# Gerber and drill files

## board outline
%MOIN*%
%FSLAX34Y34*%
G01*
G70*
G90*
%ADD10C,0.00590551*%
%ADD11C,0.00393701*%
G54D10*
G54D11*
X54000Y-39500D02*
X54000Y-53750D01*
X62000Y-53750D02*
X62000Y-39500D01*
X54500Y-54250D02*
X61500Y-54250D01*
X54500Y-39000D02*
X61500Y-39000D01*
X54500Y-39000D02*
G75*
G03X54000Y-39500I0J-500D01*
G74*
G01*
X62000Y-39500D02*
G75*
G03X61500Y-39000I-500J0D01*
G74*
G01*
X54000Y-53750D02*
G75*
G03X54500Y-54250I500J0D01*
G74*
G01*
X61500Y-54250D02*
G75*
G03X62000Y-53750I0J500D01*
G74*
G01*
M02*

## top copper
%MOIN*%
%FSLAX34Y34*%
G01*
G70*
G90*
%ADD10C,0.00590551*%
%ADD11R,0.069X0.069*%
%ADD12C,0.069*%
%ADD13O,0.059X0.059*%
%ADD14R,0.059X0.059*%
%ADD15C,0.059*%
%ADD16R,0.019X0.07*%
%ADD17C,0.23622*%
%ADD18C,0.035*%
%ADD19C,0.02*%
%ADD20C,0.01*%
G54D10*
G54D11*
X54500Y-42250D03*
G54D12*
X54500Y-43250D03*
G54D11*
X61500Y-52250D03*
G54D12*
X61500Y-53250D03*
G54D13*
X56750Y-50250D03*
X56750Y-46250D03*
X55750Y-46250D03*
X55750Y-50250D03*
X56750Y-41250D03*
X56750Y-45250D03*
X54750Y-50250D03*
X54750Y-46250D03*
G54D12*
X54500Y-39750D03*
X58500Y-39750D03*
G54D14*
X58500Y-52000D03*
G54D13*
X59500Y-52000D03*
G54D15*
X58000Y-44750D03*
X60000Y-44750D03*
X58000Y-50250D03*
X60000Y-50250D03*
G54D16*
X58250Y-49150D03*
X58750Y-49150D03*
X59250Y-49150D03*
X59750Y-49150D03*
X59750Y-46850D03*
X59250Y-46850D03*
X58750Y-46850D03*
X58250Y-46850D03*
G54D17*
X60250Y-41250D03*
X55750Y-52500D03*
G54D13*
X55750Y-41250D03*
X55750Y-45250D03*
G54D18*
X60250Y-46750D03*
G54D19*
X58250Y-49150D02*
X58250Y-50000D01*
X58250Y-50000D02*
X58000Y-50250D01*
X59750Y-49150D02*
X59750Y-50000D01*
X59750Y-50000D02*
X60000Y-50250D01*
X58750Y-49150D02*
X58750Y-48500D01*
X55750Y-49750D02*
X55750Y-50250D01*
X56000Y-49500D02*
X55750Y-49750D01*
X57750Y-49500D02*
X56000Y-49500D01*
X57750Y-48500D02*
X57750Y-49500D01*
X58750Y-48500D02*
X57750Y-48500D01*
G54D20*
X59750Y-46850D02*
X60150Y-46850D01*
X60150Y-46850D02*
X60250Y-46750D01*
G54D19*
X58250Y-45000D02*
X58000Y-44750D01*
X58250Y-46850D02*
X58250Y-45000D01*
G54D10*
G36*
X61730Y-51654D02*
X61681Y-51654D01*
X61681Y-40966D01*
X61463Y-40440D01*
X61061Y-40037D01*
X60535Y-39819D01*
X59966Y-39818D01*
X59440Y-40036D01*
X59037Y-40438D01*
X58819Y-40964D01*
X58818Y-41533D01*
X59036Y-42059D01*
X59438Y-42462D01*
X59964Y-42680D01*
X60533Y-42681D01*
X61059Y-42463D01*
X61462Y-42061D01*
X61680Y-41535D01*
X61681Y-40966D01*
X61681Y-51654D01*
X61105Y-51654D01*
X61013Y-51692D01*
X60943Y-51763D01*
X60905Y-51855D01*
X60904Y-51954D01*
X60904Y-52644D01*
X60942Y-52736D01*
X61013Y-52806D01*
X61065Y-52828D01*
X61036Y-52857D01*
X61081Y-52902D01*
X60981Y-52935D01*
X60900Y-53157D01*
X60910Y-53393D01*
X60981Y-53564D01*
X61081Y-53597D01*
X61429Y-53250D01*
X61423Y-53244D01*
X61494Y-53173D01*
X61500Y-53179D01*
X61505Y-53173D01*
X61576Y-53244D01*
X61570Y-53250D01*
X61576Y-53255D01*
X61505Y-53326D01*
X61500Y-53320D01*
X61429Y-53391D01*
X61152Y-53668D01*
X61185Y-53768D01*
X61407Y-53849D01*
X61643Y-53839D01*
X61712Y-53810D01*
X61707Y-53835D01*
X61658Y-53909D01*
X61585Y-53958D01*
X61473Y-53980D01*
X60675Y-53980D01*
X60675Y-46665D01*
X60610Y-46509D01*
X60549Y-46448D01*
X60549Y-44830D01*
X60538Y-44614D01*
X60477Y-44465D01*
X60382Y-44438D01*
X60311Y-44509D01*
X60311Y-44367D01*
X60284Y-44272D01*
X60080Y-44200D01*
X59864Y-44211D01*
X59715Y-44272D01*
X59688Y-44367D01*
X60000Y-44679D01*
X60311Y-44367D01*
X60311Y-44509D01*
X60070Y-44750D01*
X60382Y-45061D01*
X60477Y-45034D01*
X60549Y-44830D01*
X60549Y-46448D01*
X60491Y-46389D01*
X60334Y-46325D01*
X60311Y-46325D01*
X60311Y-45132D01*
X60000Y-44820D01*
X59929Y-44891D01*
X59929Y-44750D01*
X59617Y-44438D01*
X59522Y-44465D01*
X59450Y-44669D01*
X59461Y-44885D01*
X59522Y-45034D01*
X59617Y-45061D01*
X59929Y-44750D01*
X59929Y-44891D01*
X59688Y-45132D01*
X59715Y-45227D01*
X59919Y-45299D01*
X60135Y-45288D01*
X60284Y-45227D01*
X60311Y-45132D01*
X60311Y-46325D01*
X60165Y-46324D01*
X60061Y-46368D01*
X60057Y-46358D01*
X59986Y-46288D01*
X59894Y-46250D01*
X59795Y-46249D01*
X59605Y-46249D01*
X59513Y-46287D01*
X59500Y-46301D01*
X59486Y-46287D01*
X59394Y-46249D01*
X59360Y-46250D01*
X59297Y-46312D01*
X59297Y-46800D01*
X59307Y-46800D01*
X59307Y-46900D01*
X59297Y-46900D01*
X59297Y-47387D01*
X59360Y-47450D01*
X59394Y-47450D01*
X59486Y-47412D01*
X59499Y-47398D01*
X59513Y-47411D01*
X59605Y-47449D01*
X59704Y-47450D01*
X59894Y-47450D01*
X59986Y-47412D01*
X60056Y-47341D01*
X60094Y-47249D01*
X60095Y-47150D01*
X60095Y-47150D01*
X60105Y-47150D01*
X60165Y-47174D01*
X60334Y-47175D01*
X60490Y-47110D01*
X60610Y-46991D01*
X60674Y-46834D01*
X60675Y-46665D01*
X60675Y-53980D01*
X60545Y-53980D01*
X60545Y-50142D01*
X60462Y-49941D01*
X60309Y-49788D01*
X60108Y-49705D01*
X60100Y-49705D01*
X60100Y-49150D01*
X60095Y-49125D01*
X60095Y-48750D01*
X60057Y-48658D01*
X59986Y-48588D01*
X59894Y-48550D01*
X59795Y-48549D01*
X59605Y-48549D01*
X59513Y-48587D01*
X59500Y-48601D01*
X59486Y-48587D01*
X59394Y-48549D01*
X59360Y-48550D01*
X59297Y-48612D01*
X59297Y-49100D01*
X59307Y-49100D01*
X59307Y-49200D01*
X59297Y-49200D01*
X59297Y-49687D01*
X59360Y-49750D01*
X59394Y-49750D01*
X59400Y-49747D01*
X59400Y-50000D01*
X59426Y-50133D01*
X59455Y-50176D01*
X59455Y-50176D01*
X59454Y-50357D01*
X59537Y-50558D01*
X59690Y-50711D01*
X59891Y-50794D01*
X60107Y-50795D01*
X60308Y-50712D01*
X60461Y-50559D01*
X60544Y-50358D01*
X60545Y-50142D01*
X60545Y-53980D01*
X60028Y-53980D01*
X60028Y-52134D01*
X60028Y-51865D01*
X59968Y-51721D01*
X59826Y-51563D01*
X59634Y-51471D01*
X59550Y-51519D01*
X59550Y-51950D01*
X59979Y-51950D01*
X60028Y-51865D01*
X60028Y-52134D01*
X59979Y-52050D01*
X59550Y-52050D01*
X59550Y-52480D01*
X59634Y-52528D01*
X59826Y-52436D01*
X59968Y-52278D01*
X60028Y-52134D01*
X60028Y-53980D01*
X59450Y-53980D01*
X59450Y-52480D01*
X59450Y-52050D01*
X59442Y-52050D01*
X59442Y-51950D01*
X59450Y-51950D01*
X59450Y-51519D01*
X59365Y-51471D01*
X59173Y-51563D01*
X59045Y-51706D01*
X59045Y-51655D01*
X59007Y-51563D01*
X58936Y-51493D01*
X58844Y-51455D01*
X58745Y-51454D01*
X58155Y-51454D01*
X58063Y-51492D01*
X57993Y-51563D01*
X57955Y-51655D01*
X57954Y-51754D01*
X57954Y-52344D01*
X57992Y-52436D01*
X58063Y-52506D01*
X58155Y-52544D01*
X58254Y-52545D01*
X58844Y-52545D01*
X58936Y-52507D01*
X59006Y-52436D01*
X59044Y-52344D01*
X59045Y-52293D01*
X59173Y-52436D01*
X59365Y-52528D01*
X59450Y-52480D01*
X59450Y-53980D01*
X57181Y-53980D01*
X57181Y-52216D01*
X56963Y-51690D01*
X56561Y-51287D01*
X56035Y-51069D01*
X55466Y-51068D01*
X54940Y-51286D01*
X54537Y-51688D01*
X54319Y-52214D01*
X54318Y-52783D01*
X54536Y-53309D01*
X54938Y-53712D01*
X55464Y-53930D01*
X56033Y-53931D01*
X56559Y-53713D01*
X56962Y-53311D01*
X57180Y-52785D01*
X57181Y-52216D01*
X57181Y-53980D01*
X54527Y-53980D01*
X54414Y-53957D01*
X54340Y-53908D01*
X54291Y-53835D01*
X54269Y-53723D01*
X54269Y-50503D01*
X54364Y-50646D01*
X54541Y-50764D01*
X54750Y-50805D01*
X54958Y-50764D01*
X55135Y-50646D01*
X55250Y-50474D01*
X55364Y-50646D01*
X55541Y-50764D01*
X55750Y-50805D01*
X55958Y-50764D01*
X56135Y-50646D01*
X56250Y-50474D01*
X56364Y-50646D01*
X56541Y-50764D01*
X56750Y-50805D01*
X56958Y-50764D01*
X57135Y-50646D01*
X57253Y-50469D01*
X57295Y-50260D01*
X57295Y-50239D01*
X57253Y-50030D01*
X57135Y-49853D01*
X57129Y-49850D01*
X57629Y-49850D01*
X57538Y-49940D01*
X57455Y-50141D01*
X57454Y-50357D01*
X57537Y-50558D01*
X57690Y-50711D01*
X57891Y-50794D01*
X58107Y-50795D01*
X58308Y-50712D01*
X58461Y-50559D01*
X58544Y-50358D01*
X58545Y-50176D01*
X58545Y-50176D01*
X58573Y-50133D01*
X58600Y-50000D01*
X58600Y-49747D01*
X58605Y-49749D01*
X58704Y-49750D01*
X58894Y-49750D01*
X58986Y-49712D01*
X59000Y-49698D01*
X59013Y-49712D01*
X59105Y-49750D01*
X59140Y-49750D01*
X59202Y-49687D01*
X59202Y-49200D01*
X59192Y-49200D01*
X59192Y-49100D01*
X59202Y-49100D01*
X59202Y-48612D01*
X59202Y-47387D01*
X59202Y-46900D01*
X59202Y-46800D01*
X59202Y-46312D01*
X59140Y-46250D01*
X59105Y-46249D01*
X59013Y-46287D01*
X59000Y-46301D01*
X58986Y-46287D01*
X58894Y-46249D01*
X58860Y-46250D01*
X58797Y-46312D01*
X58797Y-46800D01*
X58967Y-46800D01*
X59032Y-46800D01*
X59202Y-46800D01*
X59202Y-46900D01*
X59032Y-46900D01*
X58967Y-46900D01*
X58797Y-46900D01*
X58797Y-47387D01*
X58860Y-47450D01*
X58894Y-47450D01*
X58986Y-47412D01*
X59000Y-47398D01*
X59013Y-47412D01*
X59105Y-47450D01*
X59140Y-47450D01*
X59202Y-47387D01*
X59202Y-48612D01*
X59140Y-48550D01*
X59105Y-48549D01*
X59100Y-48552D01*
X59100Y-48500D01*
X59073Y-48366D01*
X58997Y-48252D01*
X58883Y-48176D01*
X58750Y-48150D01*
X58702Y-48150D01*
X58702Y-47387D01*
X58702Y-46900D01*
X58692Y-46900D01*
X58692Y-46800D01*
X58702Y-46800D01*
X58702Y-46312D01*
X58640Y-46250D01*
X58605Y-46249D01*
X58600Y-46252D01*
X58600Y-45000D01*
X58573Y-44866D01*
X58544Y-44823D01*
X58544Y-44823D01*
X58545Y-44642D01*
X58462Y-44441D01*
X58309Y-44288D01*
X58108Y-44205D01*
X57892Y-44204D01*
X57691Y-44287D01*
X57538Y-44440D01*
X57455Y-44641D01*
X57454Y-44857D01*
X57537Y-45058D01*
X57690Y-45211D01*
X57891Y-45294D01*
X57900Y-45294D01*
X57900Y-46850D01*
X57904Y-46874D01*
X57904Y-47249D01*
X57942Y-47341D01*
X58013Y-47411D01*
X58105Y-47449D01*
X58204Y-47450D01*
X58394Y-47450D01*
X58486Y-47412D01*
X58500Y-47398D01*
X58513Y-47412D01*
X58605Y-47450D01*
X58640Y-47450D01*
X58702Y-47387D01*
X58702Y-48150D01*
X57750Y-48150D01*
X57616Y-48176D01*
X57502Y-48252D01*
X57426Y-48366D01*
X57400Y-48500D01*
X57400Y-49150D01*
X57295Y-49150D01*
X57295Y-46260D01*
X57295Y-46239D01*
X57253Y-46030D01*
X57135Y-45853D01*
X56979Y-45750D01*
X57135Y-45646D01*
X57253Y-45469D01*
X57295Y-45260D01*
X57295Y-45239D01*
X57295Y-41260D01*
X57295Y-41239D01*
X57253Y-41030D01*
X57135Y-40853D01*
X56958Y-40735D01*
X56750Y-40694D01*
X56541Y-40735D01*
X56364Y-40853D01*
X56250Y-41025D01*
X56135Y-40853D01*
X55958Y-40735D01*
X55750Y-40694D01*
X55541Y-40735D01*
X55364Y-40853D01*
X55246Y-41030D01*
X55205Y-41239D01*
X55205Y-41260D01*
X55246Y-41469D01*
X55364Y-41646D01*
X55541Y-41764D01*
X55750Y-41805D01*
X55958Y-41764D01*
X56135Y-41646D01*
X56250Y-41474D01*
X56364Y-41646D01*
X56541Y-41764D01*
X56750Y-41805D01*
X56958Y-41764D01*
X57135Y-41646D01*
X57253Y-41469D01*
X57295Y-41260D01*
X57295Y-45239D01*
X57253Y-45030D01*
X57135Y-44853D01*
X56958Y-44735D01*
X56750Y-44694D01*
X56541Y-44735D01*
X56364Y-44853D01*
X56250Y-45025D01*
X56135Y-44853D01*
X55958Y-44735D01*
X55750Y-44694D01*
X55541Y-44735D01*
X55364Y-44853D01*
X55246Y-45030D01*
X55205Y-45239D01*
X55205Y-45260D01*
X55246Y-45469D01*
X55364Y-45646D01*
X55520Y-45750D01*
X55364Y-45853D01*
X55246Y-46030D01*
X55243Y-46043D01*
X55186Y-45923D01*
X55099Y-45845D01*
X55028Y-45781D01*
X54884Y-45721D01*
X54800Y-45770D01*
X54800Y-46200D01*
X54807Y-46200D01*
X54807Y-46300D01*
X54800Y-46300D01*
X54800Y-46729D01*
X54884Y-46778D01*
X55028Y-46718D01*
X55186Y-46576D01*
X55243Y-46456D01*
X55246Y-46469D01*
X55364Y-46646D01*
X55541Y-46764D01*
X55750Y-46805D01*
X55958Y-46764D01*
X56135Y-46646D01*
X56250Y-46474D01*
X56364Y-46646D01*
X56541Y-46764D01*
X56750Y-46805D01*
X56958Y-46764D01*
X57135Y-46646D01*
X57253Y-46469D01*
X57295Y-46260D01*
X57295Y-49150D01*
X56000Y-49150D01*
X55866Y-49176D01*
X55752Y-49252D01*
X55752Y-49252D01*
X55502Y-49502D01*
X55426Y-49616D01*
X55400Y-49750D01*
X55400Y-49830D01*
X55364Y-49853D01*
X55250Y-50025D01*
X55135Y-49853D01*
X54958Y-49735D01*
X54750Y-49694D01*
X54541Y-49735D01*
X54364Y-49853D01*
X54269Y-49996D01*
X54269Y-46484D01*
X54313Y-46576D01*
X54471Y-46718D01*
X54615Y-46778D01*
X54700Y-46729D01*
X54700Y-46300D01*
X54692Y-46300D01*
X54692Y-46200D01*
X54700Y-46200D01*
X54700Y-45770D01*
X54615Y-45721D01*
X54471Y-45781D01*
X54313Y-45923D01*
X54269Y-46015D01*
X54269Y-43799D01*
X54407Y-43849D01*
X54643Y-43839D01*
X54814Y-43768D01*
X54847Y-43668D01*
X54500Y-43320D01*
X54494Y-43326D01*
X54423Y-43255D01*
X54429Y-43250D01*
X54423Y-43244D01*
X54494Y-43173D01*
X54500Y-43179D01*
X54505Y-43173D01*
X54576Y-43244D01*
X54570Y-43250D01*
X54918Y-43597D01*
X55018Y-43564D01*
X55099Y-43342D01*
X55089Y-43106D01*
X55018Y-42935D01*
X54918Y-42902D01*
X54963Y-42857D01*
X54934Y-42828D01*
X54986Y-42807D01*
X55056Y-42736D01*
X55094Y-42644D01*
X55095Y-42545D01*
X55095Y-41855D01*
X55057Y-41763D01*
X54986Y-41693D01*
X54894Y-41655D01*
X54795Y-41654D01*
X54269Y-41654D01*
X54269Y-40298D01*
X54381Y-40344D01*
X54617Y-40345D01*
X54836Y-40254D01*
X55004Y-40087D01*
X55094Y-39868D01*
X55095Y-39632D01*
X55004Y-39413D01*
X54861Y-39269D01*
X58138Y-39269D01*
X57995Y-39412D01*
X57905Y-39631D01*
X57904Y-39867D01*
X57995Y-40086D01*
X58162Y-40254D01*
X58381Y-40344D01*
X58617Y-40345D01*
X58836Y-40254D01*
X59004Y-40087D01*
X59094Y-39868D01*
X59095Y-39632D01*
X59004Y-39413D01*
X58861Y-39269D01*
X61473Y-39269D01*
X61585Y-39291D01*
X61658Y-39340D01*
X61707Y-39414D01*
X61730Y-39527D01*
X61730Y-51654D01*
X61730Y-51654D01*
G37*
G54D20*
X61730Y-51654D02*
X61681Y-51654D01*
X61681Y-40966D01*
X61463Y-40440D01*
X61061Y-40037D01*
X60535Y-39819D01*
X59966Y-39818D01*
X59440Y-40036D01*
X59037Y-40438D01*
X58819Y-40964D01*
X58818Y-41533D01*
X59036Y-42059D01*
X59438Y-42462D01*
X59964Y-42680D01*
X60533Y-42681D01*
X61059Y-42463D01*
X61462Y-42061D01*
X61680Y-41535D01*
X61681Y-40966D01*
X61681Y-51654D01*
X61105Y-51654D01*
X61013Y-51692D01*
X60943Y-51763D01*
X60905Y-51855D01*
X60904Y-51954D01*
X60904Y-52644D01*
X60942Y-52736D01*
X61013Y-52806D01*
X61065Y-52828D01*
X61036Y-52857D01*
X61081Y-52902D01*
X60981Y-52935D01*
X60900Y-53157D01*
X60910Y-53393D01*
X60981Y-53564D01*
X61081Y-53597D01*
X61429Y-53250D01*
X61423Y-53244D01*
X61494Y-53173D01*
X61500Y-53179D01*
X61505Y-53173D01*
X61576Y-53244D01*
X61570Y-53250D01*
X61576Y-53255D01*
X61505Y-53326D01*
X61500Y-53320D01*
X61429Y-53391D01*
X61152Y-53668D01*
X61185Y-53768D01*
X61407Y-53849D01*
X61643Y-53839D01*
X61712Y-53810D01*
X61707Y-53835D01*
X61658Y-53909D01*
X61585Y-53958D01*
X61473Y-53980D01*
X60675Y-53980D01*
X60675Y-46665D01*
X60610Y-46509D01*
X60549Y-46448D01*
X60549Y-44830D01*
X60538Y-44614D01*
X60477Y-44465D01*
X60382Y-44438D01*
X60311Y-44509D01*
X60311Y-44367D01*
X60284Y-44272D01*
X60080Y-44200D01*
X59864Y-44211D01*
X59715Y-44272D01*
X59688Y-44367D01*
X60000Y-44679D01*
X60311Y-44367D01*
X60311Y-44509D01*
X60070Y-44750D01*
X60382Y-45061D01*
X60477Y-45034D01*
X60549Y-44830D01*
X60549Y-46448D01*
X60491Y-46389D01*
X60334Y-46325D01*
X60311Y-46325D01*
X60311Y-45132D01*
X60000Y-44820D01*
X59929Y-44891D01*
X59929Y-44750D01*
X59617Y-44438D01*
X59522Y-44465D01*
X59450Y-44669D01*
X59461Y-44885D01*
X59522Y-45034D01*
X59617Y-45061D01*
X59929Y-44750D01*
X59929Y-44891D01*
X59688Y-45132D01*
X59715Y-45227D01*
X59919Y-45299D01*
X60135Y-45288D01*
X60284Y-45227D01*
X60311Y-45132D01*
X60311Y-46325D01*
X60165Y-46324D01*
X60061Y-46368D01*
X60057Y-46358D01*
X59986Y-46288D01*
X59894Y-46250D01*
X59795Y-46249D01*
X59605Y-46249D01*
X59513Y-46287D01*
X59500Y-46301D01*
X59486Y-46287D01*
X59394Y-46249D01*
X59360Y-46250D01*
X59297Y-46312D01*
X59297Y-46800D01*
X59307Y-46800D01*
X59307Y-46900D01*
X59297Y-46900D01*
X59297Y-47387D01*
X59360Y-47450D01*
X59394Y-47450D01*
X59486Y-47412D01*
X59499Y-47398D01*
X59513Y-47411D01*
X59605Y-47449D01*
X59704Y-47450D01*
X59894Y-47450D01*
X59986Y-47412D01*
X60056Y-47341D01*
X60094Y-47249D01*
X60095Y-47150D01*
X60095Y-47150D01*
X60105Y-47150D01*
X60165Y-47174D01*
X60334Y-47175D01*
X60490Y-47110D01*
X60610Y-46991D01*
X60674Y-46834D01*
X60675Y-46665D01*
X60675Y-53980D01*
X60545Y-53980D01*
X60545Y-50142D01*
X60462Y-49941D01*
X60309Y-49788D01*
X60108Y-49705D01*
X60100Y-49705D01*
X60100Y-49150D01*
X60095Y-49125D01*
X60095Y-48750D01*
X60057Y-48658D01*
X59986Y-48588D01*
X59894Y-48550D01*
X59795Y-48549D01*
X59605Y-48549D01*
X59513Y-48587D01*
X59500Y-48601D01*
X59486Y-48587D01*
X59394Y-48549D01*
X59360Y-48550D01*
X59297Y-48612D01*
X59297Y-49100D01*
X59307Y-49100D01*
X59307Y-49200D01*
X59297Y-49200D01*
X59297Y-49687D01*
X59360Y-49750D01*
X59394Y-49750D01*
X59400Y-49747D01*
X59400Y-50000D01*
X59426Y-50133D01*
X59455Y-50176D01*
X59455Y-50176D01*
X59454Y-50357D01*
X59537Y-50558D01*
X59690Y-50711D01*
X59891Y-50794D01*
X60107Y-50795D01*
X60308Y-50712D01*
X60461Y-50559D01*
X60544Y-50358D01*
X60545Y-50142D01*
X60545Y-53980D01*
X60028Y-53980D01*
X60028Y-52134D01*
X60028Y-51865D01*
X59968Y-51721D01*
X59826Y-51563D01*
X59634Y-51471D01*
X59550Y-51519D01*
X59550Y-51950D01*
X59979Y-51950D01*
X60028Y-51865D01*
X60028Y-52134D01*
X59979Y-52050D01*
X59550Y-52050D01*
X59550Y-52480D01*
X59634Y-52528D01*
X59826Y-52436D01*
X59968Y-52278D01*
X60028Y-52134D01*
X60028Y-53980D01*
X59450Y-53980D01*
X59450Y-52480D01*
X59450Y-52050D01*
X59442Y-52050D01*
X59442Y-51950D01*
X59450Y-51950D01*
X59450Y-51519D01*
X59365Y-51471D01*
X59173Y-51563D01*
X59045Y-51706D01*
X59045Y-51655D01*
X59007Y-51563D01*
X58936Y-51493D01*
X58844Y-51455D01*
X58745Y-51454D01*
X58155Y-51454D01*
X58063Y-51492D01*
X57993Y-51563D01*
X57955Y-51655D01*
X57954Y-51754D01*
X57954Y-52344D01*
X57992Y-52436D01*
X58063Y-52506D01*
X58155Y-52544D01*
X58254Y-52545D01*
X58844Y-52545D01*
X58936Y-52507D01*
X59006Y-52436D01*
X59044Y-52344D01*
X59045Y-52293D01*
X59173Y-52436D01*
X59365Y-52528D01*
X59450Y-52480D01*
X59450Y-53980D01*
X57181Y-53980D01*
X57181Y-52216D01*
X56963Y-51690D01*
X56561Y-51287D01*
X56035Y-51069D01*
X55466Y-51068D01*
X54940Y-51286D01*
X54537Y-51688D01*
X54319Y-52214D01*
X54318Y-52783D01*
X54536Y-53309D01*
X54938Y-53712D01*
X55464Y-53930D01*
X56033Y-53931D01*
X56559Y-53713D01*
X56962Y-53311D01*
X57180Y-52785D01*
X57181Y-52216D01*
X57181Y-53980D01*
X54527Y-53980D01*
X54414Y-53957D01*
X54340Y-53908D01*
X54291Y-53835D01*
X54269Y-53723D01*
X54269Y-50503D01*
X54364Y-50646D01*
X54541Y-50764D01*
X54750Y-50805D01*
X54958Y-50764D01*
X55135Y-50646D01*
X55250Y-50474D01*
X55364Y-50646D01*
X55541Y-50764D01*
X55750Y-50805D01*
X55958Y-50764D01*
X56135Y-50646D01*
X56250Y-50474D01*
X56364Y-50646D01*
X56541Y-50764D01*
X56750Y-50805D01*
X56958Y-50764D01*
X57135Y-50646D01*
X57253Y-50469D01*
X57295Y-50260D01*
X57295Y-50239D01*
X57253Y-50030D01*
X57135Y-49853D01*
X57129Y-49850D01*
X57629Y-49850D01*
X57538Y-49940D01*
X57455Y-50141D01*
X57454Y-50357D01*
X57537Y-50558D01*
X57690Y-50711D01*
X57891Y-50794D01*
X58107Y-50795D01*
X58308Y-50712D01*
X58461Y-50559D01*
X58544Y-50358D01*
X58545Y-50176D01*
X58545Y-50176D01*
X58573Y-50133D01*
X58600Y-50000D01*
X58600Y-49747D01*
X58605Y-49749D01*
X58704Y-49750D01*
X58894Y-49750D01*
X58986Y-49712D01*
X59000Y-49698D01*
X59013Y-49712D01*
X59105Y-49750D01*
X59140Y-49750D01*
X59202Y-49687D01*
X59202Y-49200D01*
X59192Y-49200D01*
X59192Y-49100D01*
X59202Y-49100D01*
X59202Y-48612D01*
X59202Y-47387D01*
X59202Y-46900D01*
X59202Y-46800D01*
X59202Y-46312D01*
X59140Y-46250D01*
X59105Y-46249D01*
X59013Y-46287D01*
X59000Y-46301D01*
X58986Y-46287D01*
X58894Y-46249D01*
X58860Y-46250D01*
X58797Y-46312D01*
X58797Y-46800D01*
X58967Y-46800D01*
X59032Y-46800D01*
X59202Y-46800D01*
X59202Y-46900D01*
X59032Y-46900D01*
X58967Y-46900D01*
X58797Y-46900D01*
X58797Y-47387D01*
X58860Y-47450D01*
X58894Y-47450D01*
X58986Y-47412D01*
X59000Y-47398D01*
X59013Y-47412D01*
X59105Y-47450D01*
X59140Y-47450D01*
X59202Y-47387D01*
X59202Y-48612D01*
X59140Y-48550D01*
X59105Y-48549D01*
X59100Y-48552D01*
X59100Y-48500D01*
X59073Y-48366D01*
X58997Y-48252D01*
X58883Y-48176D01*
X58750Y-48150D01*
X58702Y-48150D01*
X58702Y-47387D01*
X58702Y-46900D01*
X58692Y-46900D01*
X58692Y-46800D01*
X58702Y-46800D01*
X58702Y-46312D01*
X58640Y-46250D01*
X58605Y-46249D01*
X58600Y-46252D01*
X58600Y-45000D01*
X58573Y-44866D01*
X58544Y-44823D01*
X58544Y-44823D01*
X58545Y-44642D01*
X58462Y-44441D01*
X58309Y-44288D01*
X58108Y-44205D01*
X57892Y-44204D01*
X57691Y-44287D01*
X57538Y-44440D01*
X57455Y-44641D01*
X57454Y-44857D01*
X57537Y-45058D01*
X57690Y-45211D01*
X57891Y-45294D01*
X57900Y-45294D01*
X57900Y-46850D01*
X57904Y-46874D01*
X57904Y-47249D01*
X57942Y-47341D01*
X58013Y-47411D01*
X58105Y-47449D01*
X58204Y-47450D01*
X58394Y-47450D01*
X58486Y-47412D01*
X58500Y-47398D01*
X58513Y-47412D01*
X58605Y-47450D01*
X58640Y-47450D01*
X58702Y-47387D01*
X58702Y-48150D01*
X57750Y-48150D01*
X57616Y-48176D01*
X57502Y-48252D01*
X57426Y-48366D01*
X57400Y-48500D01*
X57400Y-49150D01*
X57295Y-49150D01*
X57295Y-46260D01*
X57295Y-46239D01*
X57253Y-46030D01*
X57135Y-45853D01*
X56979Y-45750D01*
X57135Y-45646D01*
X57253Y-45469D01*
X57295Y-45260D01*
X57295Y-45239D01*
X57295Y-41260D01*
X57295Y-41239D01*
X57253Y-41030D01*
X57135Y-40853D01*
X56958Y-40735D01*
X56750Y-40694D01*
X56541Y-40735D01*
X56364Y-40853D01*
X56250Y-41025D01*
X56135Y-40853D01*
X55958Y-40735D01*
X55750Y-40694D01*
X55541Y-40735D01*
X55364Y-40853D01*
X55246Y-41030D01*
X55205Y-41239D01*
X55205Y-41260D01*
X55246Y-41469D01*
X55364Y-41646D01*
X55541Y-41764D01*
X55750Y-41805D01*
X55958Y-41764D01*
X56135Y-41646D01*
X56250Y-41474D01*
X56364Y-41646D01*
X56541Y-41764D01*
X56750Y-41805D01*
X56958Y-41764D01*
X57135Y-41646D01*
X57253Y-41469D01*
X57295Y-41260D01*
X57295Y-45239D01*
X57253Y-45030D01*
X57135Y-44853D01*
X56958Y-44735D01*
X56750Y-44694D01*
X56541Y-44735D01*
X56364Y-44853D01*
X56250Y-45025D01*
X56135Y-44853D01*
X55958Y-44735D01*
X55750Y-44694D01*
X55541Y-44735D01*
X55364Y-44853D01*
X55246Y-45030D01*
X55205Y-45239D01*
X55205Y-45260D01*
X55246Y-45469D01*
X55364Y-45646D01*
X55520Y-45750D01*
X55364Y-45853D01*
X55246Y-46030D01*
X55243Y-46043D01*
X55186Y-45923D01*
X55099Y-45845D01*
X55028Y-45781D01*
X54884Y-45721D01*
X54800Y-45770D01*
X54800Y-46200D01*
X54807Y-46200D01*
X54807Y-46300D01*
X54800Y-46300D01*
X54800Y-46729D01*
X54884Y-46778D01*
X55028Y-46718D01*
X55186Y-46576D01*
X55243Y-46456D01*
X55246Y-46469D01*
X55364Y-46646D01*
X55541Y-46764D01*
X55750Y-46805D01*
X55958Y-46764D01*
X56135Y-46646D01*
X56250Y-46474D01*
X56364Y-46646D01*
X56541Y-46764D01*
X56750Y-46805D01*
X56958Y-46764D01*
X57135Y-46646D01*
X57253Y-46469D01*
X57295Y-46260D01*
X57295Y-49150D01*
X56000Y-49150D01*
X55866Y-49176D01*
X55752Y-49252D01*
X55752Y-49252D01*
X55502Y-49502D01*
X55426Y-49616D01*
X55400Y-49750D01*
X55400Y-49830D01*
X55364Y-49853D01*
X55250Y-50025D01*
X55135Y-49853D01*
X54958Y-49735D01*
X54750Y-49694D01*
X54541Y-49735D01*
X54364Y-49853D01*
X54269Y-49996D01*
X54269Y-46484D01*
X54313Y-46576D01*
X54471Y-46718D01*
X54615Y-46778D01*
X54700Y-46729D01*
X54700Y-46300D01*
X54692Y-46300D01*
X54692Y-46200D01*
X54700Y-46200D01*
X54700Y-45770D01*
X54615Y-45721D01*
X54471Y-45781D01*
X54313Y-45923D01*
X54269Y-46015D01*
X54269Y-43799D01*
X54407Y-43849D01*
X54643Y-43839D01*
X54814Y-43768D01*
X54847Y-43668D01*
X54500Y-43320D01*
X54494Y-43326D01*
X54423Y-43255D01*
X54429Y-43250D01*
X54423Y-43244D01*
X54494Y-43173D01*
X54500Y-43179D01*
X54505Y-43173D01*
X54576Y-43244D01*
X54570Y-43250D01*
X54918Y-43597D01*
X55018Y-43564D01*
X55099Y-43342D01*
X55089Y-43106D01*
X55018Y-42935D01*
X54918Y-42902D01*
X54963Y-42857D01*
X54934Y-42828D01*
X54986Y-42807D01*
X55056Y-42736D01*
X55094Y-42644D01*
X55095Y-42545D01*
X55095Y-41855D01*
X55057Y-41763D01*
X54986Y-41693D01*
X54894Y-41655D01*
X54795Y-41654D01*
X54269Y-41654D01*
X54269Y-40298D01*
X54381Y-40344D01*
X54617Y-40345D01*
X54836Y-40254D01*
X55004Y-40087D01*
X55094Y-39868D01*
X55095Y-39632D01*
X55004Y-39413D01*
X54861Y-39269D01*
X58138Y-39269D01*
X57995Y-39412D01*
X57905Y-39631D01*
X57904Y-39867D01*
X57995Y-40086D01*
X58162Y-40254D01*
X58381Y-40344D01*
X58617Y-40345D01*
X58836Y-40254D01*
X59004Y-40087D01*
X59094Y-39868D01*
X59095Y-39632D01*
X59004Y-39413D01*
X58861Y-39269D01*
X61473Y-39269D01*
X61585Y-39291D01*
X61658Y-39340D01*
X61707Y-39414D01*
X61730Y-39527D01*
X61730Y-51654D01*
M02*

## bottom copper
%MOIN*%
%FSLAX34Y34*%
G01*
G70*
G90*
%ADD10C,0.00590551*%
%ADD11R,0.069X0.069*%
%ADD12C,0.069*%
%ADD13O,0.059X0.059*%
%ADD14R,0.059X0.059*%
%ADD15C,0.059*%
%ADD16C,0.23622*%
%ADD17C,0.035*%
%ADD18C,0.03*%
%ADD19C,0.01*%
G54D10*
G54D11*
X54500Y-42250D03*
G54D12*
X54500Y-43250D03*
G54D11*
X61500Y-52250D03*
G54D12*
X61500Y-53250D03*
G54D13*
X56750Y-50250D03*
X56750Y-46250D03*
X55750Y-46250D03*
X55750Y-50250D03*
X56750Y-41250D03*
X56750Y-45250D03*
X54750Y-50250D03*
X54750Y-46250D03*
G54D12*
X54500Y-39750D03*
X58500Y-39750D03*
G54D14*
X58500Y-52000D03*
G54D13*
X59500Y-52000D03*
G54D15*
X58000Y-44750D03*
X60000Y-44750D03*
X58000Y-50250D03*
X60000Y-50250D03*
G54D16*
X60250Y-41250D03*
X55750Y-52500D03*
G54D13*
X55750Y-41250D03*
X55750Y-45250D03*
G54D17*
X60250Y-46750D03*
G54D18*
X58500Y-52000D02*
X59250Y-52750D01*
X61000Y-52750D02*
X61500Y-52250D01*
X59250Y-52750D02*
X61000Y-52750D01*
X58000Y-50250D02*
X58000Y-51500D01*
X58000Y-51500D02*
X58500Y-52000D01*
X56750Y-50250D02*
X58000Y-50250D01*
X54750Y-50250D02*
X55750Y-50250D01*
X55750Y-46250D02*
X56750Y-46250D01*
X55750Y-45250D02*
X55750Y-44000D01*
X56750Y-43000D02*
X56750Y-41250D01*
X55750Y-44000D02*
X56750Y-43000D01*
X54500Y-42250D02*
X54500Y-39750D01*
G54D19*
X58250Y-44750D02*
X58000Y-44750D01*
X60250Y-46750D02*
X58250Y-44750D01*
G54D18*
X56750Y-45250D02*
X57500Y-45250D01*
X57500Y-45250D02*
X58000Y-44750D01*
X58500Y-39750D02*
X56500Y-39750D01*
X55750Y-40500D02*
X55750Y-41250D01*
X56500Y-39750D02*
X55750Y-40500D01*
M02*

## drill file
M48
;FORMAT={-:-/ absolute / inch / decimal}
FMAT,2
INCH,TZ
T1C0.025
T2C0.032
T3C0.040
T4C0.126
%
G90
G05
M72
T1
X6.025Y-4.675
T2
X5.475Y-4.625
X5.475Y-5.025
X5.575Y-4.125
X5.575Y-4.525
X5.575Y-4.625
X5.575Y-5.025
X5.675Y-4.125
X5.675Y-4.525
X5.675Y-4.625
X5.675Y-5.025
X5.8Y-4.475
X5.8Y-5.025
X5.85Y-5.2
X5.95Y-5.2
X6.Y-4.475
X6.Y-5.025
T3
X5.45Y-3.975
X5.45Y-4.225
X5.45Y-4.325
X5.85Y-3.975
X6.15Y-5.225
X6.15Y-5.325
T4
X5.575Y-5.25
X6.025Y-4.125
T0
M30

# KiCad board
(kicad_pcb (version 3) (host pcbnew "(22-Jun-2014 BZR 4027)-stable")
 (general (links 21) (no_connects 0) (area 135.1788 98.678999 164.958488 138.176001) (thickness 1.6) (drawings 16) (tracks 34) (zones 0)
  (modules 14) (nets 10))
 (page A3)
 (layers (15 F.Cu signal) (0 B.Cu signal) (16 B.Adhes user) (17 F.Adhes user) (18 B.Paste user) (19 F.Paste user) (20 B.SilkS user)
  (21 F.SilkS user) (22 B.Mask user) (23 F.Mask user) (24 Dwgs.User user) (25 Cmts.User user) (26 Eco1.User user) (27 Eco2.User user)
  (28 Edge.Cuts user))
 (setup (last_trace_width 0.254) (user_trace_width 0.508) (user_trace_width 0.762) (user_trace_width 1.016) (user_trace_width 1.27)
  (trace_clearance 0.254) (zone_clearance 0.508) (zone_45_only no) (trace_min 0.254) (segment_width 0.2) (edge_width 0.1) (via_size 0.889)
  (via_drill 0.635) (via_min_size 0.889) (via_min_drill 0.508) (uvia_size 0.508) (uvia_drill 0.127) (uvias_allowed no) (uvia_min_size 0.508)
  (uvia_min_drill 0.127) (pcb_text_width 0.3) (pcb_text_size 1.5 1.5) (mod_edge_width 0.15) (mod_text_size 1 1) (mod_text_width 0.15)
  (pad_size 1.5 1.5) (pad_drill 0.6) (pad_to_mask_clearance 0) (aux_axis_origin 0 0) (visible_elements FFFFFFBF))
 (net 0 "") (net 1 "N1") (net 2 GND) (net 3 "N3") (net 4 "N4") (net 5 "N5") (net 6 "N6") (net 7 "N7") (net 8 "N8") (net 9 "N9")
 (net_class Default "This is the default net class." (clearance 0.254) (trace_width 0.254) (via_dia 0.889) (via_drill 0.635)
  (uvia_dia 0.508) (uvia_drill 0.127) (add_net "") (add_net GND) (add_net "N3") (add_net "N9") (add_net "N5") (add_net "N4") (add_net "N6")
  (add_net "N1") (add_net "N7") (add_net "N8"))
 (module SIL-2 (layer F.Cu) (at 138.43 107.315 270)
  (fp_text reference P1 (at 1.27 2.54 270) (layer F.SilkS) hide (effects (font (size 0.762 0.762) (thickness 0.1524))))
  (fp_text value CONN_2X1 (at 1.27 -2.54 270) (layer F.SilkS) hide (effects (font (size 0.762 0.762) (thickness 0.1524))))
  (pad 1 thru_hole rect (at 0 0 270) (size 1.7526 1.7526) (drill 1.016) (layers *.Cu *.Mask F.SilkS) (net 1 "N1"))
  (pad 2 thru_hole circle (at 2.54 0 270) (size 1.7526 1.7526) (drill 1.016) (layers *.Cu *.Mask F.SilkS) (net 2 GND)))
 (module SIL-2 (layer F.Cu) (at 156.21 132.715 270)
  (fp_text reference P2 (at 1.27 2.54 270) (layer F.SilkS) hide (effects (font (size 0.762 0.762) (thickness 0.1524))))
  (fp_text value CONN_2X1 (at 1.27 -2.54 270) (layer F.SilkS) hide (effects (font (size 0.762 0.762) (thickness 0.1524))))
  (pad 1 thru_hole rect (at 0 0 270) (size 1.7526 1.7526) (drill 1.016) (layers *.Cu *.Mask F.SilkS) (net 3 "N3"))
  (pad 2 thru_hole circle (at 2.54 0 270) (size 1.7526 1.7526) (drill 1.016) (layers *.Cu *.Mask F.SilkS) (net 2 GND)))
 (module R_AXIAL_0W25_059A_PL (layer F.Cu) (at 144.145 127.635 90) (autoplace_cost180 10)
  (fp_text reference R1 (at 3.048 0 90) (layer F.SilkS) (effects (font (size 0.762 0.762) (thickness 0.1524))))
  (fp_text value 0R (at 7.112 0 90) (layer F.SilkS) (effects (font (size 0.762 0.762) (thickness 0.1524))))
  (pad 1 thru_hole oval (at 0 0 90) (size 1.4986 1.4986) (drill 0.8128) (layers *.Cu *.Mask F.SilkS) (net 3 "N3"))
  (pad 2 thru_hole oval (at 10.16 0 90) (size 1.4986 1.4986) (drill 0.8128) (layers *.Cu *.Mask F.SilkS) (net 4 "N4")))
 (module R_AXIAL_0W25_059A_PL (layer F.Cu) (at 141.605 117.475 270) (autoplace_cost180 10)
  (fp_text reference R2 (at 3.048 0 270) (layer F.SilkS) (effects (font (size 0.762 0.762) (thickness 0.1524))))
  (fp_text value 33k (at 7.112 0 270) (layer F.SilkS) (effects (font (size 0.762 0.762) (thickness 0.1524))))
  (pad 1 thru_hole oval (at 0 0 270) (size 1.4986 1.4986) (drill 0.8128) (layers *.Cu *.Mask F.SilkS) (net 4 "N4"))
  (pad 2 thru_hole oval (at 10.16 0 270) (size 1.4986 1.4986) (drill 0.8128) (layers *.Cu *.Mask F.SilkS) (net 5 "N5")))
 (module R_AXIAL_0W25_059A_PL (layer F.Cu) (at 144.145 104.775 270) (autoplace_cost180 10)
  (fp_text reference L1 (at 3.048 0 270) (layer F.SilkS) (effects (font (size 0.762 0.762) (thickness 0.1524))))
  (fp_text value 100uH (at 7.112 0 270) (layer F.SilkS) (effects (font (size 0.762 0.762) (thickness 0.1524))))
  (pad 1 thru_hole oval (at 0 0 270) (size 1.4986 1.4986) (drill 0.8128) (layers *.Cu *.Mask F.SilkS) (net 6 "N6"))
  (pad 2 thru_hole oval (at 10.16 0 270) (size 1.4986 1.4986) (drill 0.8128) (layers *.Cu *.Mask F.SilkS) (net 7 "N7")))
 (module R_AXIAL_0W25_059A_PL (layer F.Cu) (at 139.065 127.635 90) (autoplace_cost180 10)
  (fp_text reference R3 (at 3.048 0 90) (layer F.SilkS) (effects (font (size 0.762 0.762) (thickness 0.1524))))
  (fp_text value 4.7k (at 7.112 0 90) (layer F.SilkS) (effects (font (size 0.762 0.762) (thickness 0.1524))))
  (pad 1 thru_hole oval (at 0 0 90) (size 1.4986 1.4986) (drill 0.8128) (layers *.Cu *.Mask F.SilkS) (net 5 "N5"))
  (pad 2 thru_hole oval (at 10.16 0 90) (size 1.4986 1.4986) (drill 0.8128) (layers *.Cu *.Mask F.SilkS) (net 2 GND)))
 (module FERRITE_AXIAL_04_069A (layer F.Cu) (at 143.51 100.965)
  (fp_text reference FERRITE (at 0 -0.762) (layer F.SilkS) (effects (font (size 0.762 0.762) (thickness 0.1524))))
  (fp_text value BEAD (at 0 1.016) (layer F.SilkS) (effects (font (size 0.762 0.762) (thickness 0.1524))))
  (pad 1 thru_hole circle (at -5.08 0) (size 1.7526 1.7526) (drill 1.016) (layers *.Cu *.Mask F.SilkS) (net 1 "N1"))
  (pad 2 thru_hole circle (at 5.08 0) (size 1.7526 1.7526) (drill 1.016) (layers *.Cu *.Mask F.SilkS) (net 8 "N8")))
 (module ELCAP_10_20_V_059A (layer F.Cu) (at 148.59 132.08)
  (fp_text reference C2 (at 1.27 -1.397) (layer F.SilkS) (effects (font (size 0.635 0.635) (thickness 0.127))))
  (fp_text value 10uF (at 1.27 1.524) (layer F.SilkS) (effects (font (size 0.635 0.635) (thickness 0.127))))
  (pad 1 thru_hole rect (at 0 0) (size 1.4986 1.4986) (drill 0.8128) (layers *.Cu *.Mask F.SilkS) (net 3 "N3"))
  (pad 2 thru_hole oval (at 2.54 0) (size 1.4986 1.4986) (drill 0.8128) (layers *.Cu *.Mask F.SilkS) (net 2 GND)))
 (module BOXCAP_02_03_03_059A (layer F.Cu) (at 149.86 113.665)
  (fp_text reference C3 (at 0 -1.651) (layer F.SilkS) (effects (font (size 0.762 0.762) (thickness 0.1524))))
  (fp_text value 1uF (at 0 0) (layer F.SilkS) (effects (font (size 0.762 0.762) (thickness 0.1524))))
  (pad 1 thru_hole circle (at -2.54 0) (size 1.4986 1.4986) (drill 0.8128) (layers *.Cu *.Mask F.SilkS) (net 7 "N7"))
  (pad 2 thru_hole circle (at 2.54 0) (size 1.4986 1.4986) (drill 0.8128) (layers *.Cu *.Mask F.SilkS) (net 2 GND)))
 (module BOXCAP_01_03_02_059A (layer F.Cu) (at 149.86 127.635)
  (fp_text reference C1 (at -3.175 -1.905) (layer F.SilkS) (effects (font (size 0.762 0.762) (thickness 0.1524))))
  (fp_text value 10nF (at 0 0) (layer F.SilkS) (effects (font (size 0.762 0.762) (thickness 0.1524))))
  (pad 1 thru_hole circle (at -2.54 0) (size 1.4986 1.4986) (drill 0.8128) (layers *.Cu *.Mask F.SilkS) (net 3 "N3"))
  (pad 2 thru_hole circle (at 2.54 0) (size 1.4986 1.4986) (drill 0.8128) (layers *.Cu *.Mask F.SilkS) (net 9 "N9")))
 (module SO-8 (layer F.Cu) (at 149.86 121.92)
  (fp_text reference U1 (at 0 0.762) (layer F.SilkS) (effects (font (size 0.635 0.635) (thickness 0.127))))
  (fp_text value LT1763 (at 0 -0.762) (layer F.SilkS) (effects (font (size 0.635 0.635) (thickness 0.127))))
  (pad 1 smd rect (at -1.905 2.921) (size 0.4826 1.778) (layers F.Cu F.Paste F.Mask) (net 3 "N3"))
  (pad 2 smd rect (at -0.635 2.921) (size 0.4826 1.778) (layers F.Cu F.Paste F.Mask) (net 5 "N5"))
  (pad 3 smd rect (at 0.635 2.921) (size 0.4826 1.778) (layers F.Cu F.Paste F.Mask) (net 2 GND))
  (pad 4 smd rect (at 1.905 2.921) (size 0.4826 1.778) (layers F.Cu F.Paste F.Mask) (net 9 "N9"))
  (pad 5 smd rect (at 1.905 -2.921) (size 0.4826 1.778) (layers F.Cu F.Paste F.Mask) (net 7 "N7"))
  (pad 6 smd rect (at 0.635 -2.921) (size 0.4826 1.778) (layers F.Cu F.Paste F.Mask) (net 2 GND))
  (pad 7 smd rect (at -0.635 -2.921) (size 0.4826 1.778) (layers F.Cu F.Paste F.Mask) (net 2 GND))
  (pad 8 smd rect (at -1.905 -2.921) (size 0.4826 1.778) (layers F.Cu F.Paste F.Mask) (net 7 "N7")))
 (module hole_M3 (layer F.Cu) (at 153.035 104.775)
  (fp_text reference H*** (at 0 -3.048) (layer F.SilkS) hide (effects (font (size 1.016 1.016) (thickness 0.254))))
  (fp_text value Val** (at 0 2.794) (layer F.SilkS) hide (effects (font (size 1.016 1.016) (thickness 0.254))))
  (pad 1 thru_hole circle (at 0 0) (size 6 6) (drill 3.2) (layers *.Cu *.Mask F.SilkS)))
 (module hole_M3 (layer F.Cu) (at 141.605 133.35)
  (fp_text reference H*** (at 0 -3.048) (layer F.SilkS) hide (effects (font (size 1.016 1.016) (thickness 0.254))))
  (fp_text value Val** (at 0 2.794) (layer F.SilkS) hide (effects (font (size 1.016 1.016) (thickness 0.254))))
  (pad 1 thru_hole circle (at 0 0) (size 6 6) (drill 3.2) (layers *.Cu *.Mask F.SilkS)))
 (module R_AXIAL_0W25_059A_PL (layer F.Cu) (at 141.605 104.775 270) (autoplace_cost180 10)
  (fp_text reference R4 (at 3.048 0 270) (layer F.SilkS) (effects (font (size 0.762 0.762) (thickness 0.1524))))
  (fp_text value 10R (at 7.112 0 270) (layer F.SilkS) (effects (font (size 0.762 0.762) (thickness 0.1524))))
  (pad 1 thru_hole oval (at 0 0 270) (size 1.4986 1.4986) (drill 0.8128) (layers *.Cu *.Mask F.SilkS) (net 8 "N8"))
  (pad 2 thru_hole oval (at 10.16 0 270) (size 1.4986 1.4986) (drill 0.8128) (layers *.Cu *.Mask F.SilkS) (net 6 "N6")))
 (gr_line (start 137.16 100.33) (end 137.16 136.525) (angle 90) (layer Edge.Cuts) (width 0.1))
 (gr_line (start 157.48 136.525) (end 157.48 100.33) (angle 90) (layer Edge.Cuts) (width 0.1))
 (gr_line (start 138.43 137.795) (end 156.21 137.795) (angle 90) (layer Edge.Cuts) (width 0.1))
 (gr_line (start 138.43 99.06) (end 156.21 99.06) (angle 90) (layer Edge.Cuts) (width 0.1))
 (gr_arc (start 138.43 100.33) (end 137.16 100.33) (angle 90) (layer Edge.Cuts) (width 0.1))
 (gr_arc (start 156.21 100.33) (end 156.21 99.06) (angle 90) (layer Edge.Cuts) (width 0.1))
 (gr_arc (start 138.43 136.525) (end 138.43 137.795) (angle 90) (layer Edge.Cuts) (width 0.1))
 (gr_arc (start 156.21 136.525) (end 157.48 136.525) (angle 90) (layer Edge.Cuts) (width 0.1))
 (segment (start 148.59 132.08) (end 150.495 133.985) (width 0.762) (layer B.Cu) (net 3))
 (segment (start 154.94 133.985) (end 156.21 132.715) (width 0.762) (layer B.Cu) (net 3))
 (segment (start 150.495 133.985) (end 154.94 133.985) (width 0.762) (layer B.Cu) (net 3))
 (segment (start 147.955 124.841) (end 147.955 127) (width 0.508) (layer F.Cu) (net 3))
 (segment (start 147.955 127) (end 147.32 127.635) (width 0.508) (layer F.Cu) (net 3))
 (segment (start 147.32 127.635) (end 147.32 130.81) (width 0.762) (layer B.Cu) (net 3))
 (segment (start 147.32 130.81) (end 148.59 132.08) (width 0.762) (layer B.Cu) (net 3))
 (segment (start 144.145 127.635) (end 147.32 127.635) (width 0.762) (layer B.Cu) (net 3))
 (segment (start 151.765 124.841) (end 151.765 127) (width 0.508) (layer F.Cu) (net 9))
 (segment (start 151.765 127) (end 152.4 127.635) (width 0.508) (layer F.Cu) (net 9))
 (segment (start 149.225 124.841) (end 149.225 123.19) (width 0.508) (layer F.Cu) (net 5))
 (segment (start 141.605 126.365) (end 141.605 127.635) (width 0.508) (layer F.Cu) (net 5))
 (segment (start 142.24 125.73) (end 141.605 126.365) (width 0.508) (layer F.Cu) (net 5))
 (segment (start 146.685 125.73) (end 142.24 125.73) (width 0.508) (layer F.Cu) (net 5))
 (segment (start 146.685 123.19) (end 146.685 125.73) (width 0.508) (layer F.Cu) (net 5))
 (segment (start 149.225 123.19) (end 146.685 123.19) (width 0.508) (layer F.Cu) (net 5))
 (segment (start 139.065 127.635) (end 141.605 127.635) (width 0.762) (layer B.Cu) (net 5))
 (segment (start 141.605 117.475) (end 144.145 117.475) (width 0.762) (layer B.Cu) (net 4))
 (segment (start 141.605 114.935) (end 141.605 111.76) (width 0.762) (layer B.Cu) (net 6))
 (segment (start 144.145 109.22) (end 144.145 104.775) (width 0.762) (layer B.Cu) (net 6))
 (segment (start 141.605 111.76) (end 144.145 109.22) (width 0.762) (layer B.Cu) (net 6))
 (segment (start 138.43 107.315) (end 138.43 100.965) (width 0.762) (layer B.Cu) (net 1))
 (segment (start 151.765 118.999) (end 152.781 118.999) (width 0.254) (layer F.Cu) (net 7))
 (segment (start 147.955 113.665) (end 147.32 113.665) (width 0.254) (layer B.Cu) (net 7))
 (segment (start 153.035 118.745) (end 147.955 113.665) (width 0.254) (layer B.Cu) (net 7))
 (via (at 153.035 118.745) (size 0.889) (layers F.Cu B.Cu) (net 7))
 (segment (start 152.781 118.999) (end 153.035 118.745) (width 0.254) (layer F.Cu) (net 7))
 (segment (start 147.955 114.3) (end 147.32 113.665) (width 0.508) (layer F.Cu) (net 7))
 (segment (start 147.955 118.999) (end 147.955 114.3) (width 0.508) (layer F.Cu) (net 7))
 (segment (start 144.145 114.935) (end 146.05 114.935) (width 0.762) (layer B.Cu) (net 7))
 (segment (start 146.05 114.935) (end 147.32 113.665) (width 0.762) (layer B.Cu) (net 7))
 (segment (start 148.59 100.965) (end 143.51 100.965) (width 0.762) (layer B.Cu) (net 8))
 (segment (start 141.605 102.87) (end 141.605 104.775) (width 0.762) (layer B.Cu) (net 8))
 (segment (start 143.51 100.965) (end 141.605 102.87) (width 0.762) (layer B.Cu) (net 8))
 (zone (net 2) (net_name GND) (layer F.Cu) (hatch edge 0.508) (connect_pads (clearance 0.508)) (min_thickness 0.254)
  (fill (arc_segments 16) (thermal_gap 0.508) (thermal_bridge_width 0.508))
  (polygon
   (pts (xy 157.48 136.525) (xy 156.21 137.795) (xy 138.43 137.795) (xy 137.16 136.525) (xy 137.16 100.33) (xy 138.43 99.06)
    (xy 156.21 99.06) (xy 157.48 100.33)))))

